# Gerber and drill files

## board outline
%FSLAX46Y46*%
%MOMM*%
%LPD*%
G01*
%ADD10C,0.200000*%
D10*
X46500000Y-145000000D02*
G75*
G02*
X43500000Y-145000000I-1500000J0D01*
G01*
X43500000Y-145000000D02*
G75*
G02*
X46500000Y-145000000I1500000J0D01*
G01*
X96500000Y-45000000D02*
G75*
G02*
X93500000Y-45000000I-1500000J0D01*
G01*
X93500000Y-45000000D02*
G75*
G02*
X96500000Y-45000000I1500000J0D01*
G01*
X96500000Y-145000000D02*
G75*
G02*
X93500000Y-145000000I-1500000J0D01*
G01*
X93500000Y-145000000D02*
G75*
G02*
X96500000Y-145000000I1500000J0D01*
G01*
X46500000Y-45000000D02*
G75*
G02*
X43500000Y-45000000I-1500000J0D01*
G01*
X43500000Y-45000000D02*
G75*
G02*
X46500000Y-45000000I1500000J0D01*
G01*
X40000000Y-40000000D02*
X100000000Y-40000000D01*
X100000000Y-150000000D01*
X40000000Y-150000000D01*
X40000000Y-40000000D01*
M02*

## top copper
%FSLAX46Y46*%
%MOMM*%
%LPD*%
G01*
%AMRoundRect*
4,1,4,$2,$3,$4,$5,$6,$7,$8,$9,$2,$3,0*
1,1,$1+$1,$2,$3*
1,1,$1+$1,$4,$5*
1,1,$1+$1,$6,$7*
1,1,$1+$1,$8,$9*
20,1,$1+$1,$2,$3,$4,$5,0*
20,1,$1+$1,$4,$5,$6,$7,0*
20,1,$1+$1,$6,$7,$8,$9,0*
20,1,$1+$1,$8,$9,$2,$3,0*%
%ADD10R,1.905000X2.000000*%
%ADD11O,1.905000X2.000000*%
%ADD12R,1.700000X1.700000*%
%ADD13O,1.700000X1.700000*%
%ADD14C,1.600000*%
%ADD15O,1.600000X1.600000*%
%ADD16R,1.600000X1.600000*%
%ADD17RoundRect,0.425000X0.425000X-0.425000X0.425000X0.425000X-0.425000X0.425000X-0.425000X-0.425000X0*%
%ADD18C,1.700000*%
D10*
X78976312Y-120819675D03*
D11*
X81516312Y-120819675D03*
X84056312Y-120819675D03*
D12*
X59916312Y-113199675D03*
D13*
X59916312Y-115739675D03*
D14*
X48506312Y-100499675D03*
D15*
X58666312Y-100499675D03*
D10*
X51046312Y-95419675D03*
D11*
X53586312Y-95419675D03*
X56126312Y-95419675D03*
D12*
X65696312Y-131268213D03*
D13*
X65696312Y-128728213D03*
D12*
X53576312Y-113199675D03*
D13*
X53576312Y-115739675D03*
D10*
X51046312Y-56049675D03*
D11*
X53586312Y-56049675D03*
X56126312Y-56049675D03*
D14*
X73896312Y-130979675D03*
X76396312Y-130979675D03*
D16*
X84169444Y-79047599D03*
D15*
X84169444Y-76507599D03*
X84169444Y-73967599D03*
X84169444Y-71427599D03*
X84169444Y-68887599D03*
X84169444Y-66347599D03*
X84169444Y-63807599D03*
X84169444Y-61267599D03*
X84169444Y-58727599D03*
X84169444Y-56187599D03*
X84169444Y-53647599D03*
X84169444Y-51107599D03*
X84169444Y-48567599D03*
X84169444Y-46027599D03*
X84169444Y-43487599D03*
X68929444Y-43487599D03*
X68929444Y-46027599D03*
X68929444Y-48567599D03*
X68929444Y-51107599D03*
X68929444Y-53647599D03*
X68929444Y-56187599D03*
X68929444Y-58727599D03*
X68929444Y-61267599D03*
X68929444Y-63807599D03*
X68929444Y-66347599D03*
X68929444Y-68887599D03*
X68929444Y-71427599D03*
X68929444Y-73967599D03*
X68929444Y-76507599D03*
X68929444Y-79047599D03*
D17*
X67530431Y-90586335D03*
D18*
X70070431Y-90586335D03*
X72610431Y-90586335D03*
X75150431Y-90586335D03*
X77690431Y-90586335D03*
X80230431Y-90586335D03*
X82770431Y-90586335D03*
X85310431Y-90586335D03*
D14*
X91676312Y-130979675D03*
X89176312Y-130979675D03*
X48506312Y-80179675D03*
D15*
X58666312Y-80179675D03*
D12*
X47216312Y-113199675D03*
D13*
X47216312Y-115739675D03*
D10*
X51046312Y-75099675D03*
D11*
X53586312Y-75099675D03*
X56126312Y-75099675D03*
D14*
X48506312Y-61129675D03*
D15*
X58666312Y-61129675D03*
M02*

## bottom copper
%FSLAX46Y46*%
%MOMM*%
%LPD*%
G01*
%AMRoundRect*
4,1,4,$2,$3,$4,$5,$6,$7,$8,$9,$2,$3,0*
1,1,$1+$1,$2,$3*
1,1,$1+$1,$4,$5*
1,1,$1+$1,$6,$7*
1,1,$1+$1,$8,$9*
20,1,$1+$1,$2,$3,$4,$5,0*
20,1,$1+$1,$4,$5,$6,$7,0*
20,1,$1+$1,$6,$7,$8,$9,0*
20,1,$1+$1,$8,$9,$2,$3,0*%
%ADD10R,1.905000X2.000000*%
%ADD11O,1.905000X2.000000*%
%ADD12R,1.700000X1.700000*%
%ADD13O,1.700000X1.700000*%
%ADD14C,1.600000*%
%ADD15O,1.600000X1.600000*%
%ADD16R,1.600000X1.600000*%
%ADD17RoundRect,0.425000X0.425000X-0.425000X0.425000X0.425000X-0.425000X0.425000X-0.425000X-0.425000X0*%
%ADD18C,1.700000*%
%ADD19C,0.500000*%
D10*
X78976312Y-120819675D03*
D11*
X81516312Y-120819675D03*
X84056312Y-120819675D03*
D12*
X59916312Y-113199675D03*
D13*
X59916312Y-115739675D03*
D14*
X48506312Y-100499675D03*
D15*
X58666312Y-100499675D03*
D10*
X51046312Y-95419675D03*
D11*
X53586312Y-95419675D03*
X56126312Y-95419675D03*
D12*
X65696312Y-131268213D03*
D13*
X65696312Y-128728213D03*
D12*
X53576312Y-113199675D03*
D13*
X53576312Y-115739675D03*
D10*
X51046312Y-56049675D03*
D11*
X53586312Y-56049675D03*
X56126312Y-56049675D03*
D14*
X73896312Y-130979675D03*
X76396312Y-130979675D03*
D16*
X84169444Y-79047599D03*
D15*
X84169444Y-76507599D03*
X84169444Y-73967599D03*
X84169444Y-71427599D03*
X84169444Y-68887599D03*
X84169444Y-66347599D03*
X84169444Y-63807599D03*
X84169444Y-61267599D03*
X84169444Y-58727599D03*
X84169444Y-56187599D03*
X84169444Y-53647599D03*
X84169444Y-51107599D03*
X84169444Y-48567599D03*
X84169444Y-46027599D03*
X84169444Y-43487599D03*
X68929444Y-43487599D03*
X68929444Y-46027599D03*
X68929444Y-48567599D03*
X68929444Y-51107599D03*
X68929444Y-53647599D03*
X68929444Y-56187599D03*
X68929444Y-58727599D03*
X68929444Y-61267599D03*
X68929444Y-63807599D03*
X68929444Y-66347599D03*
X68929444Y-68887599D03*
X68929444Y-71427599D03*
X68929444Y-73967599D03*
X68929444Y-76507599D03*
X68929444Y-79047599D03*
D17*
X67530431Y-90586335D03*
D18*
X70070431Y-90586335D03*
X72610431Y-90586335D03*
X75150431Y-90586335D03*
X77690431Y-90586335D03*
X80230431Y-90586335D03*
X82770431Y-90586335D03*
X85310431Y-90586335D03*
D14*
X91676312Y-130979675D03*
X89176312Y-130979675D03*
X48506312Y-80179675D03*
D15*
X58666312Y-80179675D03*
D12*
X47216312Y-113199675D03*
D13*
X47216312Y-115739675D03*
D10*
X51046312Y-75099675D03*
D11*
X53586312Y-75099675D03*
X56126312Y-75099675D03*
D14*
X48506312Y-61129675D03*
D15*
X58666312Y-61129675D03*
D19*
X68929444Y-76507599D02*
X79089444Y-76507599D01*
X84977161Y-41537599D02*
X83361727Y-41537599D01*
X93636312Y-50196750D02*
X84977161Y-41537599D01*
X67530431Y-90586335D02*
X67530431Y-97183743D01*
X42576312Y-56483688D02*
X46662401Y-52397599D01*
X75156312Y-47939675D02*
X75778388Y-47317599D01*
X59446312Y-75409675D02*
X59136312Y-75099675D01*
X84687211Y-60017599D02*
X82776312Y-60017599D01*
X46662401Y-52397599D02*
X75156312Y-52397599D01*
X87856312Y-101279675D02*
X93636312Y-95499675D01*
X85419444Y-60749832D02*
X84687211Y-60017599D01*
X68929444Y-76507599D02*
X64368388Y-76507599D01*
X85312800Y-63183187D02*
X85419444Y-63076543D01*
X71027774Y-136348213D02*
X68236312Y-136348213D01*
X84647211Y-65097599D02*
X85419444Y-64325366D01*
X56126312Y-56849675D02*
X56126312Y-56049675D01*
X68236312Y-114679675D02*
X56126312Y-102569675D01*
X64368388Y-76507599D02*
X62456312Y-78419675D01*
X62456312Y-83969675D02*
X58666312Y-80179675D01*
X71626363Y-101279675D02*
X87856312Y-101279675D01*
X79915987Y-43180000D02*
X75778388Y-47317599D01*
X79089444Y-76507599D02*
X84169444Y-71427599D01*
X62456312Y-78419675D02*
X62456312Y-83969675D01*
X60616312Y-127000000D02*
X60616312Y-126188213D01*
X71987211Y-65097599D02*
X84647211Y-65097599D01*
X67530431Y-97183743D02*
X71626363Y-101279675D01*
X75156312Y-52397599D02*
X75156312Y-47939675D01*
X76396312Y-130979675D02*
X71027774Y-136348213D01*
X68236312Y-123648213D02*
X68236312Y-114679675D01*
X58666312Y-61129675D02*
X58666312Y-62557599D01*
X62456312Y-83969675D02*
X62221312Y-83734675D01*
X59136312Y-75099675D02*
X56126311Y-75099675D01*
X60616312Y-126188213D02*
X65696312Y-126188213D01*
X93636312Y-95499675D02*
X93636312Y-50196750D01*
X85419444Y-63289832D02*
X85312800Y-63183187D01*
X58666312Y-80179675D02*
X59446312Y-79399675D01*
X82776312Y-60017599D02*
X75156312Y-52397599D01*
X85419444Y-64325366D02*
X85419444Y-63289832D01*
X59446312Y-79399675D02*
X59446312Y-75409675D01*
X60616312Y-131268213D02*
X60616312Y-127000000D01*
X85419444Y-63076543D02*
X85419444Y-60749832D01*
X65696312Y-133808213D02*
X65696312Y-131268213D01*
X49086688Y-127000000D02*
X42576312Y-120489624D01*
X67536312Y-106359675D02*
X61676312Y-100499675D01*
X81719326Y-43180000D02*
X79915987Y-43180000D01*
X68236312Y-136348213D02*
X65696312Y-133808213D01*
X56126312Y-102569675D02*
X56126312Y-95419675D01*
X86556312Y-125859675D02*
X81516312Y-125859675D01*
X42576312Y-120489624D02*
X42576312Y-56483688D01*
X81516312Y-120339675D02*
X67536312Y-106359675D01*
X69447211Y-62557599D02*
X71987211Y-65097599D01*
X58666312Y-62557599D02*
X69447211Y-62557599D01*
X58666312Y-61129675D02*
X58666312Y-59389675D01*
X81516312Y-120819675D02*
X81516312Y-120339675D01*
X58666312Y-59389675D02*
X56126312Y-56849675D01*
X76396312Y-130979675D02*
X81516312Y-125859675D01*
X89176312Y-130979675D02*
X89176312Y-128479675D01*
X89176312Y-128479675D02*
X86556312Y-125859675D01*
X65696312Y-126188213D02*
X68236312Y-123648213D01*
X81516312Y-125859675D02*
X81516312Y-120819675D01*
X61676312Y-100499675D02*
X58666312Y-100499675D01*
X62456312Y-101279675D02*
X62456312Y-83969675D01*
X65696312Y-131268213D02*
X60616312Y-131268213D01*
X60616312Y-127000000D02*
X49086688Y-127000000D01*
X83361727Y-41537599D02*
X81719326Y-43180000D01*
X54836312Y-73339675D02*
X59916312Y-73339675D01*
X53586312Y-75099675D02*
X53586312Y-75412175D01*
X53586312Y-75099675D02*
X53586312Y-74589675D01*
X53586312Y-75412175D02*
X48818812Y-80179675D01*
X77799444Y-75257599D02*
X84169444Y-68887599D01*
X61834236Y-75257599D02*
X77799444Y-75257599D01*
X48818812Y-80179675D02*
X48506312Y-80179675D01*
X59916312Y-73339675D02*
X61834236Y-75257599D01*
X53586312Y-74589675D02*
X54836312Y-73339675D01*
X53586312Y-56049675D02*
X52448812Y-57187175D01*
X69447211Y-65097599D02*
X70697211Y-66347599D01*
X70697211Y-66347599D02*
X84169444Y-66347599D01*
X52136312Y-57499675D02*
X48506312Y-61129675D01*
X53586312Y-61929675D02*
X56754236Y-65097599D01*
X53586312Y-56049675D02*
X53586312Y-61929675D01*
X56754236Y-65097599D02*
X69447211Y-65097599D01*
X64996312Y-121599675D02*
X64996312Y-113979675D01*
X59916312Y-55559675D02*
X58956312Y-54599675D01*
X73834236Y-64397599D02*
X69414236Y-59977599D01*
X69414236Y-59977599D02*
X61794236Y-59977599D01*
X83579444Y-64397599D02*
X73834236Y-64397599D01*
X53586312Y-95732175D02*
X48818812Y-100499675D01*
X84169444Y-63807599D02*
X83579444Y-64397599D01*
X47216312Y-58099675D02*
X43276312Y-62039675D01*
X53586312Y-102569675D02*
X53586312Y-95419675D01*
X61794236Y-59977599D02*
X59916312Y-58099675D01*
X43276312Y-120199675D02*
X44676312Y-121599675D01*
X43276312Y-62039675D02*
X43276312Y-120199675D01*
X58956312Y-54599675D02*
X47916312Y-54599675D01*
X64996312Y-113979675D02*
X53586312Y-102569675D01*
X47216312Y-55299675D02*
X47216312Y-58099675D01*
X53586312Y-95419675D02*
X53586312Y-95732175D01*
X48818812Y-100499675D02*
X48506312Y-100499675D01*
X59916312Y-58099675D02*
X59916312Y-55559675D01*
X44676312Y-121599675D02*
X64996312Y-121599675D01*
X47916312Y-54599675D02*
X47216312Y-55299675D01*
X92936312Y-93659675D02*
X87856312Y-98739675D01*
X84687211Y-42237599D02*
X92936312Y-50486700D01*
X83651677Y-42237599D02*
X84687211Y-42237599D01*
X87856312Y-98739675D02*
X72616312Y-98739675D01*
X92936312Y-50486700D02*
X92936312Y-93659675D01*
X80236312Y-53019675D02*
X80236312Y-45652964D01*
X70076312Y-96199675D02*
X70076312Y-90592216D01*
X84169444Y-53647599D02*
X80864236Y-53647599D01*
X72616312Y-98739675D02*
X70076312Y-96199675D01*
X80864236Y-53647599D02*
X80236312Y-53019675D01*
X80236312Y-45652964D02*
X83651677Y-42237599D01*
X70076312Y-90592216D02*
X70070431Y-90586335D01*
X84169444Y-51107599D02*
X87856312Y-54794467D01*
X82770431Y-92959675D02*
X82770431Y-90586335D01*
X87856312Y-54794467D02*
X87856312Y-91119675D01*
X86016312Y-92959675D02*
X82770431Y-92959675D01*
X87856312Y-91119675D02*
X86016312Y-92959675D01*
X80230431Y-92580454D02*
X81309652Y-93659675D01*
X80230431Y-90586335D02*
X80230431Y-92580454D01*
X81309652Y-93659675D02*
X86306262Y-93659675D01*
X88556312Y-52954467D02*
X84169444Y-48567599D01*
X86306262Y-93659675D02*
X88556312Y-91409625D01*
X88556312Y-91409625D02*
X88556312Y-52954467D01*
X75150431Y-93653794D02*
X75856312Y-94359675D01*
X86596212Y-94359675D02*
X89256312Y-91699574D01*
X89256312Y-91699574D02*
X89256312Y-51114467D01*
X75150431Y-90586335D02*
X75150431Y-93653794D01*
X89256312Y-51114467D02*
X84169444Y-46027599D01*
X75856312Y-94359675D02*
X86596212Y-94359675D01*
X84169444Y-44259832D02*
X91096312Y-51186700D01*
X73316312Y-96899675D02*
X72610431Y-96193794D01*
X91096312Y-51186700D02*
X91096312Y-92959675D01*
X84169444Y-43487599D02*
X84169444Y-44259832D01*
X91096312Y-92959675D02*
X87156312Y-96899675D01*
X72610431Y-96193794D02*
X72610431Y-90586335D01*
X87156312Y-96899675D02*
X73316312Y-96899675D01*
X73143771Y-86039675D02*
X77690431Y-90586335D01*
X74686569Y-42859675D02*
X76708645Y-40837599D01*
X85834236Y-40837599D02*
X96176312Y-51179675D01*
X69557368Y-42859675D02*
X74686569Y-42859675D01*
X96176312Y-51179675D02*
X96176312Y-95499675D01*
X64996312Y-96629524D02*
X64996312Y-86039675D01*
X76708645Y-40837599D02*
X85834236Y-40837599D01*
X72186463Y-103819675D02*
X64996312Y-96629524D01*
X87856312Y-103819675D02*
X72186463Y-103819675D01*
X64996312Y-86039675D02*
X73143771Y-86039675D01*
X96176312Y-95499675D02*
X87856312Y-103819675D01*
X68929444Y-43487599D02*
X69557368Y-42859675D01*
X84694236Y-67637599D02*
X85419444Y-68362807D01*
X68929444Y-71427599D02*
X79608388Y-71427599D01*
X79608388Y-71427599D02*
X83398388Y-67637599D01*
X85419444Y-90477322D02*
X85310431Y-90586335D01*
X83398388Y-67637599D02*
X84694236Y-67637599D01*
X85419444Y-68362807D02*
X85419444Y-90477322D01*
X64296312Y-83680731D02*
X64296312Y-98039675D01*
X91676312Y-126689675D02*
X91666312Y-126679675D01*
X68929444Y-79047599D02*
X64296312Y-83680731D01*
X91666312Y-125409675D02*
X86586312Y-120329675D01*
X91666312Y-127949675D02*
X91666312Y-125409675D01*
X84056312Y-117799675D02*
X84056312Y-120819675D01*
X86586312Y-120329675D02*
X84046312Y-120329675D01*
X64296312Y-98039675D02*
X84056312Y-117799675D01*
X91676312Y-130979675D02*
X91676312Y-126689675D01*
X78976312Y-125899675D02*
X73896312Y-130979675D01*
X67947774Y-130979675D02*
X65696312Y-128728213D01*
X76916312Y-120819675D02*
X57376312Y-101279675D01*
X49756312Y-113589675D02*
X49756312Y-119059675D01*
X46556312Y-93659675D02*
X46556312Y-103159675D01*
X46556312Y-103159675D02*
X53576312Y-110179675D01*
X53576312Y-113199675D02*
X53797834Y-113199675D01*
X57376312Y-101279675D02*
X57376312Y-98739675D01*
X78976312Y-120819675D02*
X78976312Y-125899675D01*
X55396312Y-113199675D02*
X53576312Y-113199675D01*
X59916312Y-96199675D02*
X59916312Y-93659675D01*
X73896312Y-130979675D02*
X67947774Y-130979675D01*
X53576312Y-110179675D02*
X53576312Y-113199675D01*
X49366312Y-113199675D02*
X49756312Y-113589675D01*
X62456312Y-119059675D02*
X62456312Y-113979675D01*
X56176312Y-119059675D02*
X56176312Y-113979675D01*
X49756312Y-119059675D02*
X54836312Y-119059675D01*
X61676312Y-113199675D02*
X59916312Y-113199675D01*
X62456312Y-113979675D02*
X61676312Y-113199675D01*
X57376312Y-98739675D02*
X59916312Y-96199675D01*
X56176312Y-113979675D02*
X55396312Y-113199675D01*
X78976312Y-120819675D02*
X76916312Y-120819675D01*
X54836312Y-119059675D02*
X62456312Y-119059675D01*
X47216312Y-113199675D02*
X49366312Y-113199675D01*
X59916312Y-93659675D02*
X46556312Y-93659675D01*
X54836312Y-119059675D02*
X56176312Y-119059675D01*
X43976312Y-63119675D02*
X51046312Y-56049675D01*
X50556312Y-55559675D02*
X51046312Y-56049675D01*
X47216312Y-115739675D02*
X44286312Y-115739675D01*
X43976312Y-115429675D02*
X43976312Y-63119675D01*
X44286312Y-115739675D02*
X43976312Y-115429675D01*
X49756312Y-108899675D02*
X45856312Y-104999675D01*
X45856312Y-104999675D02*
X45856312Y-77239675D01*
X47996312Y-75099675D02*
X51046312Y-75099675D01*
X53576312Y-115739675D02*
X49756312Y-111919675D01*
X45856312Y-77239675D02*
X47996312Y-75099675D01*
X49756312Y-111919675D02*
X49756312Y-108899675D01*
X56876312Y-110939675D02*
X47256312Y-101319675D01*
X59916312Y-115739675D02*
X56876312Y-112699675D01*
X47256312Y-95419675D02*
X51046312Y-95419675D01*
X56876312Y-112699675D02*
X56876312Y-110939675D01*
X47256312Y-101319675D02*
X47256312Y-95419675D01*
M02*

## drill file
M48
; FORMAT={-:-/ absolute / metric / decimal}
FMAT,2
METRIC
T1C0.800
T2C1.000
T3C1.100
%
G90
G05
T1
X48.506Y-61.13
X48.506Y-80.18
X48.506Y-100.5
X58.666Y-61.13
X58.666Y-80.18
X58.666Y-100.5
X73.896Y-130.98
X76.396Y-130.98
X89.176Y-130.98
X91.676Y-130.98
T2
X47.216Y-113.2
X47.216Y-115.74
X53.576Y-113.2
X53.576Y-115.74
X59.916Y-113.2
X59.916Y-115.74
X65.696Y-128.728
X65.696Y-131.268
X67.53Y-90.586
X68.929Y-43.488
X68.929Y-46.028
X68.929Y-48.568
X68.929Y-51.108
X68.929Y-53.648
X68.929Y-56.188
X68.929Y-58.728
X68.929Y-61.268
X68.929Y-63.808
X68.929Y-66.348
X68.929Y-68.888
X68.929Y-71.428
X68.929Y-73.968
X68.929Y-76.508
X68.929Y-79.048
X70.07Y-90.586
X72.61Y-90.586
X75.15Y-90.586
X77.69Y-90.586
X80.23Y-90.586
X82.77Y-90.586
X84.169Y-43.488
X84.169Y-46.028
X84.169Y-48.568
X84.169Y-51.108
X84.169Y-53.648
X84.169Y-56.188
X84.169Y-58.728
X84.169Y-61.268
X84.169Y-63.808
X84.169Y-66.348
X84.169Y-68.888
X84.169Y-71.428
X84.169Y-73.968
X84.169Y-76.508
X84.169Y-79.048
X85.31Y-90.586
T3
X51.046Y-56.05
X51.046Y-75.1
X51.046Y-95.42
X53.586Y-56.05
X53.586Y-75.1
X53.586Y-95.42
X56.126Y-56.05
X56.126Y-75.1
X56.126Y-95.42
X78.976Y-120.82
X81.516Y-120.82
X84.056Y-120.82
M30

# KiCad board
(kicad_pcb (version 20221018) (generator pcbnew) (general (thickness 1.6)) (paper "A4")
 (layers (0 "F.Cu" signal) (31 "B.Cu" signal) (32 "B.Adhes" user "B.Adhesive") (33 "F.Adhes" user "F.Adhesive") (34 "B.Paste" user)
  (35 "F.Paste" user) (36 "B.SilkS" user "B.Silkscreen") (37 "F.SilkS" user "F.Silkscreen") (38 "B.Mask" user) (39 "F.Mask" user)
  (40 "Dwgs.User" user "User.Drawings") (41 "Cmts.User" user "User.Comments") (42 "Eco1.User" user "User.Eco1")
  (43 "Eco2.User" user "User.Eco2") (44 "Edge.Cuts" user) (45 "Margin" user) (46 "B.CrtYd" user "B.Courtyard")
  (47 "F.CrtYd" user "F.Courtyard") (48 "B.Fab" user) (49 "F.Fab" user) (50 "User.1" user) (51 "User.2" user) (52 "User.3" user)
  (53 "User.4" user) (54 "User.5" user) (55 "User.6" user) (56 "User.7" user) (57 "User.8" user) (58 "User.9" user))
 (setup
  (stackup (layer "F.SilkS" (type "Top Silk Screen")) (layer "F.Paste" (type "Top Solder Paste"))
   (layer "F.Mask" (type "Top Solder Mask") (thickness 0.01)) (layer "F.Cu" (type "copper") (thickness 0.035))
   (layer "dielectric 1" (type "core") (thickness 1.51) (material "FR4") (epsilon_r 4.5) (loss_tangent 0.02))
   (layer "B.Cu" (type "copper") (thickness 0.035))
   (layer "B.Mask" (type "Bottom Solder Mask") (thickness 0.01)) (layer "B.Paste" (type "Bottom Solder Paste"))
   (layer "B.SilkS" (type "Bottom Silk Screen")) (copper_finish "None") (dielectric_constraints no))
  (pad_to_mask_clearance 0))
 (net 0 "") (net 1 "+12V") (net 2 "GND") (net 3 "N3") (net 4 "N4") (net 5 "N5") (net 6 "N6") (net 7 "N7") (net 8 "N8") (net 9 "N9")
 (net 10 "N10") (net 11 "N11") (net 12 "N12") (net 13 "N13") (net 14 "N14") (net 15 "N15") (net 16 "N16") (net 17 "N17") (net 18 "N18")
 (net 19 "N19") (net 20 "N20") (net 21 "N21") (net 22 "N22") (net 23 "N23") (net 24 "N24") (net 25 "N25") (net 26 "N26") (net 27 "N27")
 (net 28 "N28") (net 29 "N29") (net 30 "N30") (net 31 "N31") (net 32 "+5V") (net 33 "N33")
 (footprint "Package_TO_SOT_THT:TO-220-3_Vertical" (layer "F.Cu") (at 78.976312 120.819675)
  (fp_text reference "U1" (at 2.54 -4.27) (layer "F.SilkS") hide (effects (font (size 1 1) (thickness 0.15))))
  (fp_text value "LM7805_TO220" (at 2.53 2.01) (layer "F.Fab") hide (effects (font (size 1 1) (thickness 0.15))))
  (pad "1" thru_hole rect (at 0 0) (size 1.905 2) (drill 1.1) (layers "*.Cu" "*.Mask") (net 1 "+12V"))
  (pad "2" thru_hole oval (at 2.54 0) (size 1.905 2) (drill 1.1) (layers "*.Cu" "*.Mask") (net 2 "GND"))
  (pad "3" thru_hole oval (at 5.08 0) (size 1.905 2) (drill 1.1) (layers "*.Cu" "*.Mask") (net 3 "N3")))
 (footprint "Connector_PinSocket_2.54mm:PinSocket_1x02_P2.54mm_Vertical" (layer "F.Cu") (at 59.916312 113.199675)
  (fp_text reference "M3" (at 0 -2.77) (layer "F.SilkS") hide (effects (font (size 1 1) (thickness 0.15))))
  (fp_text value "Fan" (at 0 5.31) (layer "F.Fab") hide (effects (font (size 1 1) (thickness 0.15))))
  (pad "1" thru_hole rect (at 0 0) (size 1.7 1.7) (drill 1) (layers "*.Cu" "*.Mask") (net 1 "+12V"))
  (pad "2" thru_hole oval (at 0 2.54) (size 1.7 1.7) (drill 1) (layers "*.Cu" "*.Mask") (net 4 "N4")))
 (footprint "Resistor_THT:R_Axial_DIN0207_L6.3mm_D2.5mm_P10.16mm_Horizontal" (layer "F.Cu") (at 48.506312 100.499675)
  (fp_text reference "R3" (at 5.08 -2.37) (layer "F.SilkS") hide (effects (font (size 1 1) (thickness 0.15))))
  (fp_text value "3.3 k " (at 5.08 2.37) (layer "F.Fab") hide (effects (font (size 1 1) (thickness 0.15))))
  (pad "1" thru_hole circle (at 0 0) (size 1.6 1.6) (drill 0.8) (layers "*.Cu" "*.Mask") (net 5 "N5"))
  (pad "2" thru_hole oval (at 10.16 0) (size 1.6 1.6) (drill 0.8) (layers "*.Cu" "*.Mask") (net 2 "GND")))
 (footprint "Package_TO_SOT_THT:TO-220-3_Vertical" (layer "F.Cu") (at 51.046312 95.419675)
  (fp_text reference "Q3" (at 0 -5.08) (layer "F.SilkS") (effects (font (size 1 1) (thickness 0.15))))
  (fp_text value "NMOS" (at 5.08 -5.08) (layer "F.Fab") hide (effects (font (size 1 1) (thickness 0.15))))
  (pad "1" thru_hole rect (at 0 0) (size 1.905 2) (drill 1.1) (layers "*.Cu" "*.Mask") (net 4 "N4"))
  (pad "2" thru_hole oval (at 2.54 0) (size 1.905 2) (drill 1.1) (layers "*.Cu" "*.Mask") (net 5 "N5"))
  (pad "3" thru_hole oval (at 5.08 0) (size 1.905 2) (drill 1.1) (layers "*.Cu" "*.Mask") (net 2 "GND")))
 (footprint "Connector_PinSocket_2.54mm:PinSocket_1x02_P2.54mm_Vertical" (layer "F.Cu") (at 65.696312 131.268213 180)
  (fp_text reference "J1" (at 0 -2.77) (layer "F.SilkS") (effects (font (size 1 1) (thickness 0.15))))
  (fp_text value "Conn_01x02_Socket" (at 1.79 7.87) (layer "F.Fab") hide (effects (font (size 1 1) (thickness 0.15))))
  (pad "1" thru_hole rect (at 0 0 180) (size 1.7 1.7) (drill 1) (layers "*.Cu" "*.Mask") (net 2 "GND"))
  (pad "2" thru_hole oval (at 0 2.54 180) (size 1.7 1.7) (drill 1) (layers "*.Cu" "*.Mask") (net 1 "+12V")))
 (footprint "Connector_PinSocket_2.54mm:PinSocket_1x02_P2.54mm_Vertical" (layer "F.Cu") (at 53.576312 113.199675)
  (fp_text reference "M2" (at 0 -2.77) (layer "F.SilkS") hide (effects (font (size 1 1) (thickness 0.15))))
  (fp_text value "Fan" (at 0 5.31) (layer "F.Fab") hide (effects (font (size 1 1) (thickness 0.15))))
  (pad "1" thru_hole rect (at 0 0) (size 1.7 1.7) (drill 1) (layers "*.Cu" "*.Mask") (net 1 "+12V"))
  (pad "2" thru_hole oval (at 0 2.54) (size 1.7 1.7) (drill 1) (layers "*.Cu" "*.Mask") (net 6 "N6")))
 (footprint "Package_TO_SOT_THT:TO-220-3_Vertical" (layer "F.Cu") (at 51.046312 56.049675)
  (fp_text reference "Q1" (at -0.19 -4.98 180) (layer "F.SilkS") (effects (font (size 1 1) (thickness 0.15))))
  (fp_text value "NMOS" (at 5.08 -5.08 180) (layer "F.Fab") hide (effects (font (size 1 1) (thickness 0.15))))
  (pad "1" thru_hole rect (at 0 0) (size 1.905 2) (drill 1.1) (layers "*.Cu" "*.Mask") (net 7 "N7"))
  (pad "2" thru_hole oval (at 2.54 0) (size 1.905 2) (drill 1.1) (layers "*.Cu" "*.Mask") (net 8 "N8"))
  (pad "3" thru_hole oval (at 5.08 0) (size 1.905 2) (drill 1.1) (layers "*.Cu" "*.Mask") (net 2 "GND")))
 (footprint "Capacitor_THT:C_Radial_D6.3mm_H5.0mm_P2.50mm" (layer "F.Cu") (at 73.896312 130.979675)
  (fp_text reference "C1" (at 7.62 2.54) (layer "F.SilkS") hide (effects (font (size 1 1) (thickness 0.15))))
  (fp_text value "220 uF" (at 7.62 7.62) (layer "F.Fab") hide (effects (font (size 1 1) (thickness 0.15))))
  (pad "1" thru_hole circle (at 0 0) (size 1.6 1.6) (drill 0.8) (layers "*.Cu" "*.Mask") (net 1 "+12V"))
  (pad "2" thru_hole circle (at 2.5 0) (size 1.6 1.6) (drill 0.8) (layers "*.Cu" "*.Mask") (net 2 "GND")))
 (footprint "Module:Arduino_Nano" (layer "F.Cu") (at 84.169444 79.047599 180)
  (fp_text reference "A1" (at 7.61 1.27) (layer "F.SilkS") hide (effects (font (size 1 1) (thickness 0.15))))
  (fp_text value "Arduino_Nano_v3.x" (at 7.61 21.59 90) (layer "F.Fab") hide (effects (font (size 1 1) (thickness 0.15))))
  (pad "1" thru_hole rect (at 0 0 180) (size 1.6 1.6) (drill 1) (layers "*.Cu" "*.Mask") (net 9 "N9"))
  (pad "2" thru_hole oval (at 0 2.54 180) (size 1.6 1.6) (drill 1) (layers "*.Cu" "*.Mask") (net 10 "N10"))
  (pad "3" thru_hole oval (at 0 5.08 180) (size 1.6 1.6) (drill 1) (layers "*.Cu" "*.Mask") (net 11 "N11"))
  (pad "4" thru_hole oval (at 0 7.62 180) (size 1.6 1.6) (drill 1) (layers "*.Cu" "*.Mask") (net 2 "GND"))
  (pad "5" thru_hole oval (at 0 10.16 180) (size 1.6 1.6) (drill 1) (layers "*.Cu" "*.Mask") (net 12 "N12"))
  (pad "6" thru_hole oval (at 0 12.7 180) (size 1.6 1.6) (drill 1) (layers "*.Cu" "*.Mask") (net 8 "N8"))
  (pad "7" thru_hole oval (at 0 15.24 180) (size 1.6 1.6) (drill 1) (layers "*.Cu" "*.Mask") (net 5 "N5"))
  (pad "8" thru_hole oval (at 0 17.78 180) (size 1.6 1.6) (drill 1) (layers "*.Cu" "*.Mask") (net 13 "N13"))
  (pad "9" thru_hole oval (at 0 20.32 180) (size 1.6 1.6) (drill 1) (layers "*.Cu" "*.Mask") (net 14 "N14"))
  (pad "10" thru_hole oval (at 0 22.86 180) (size 1.6 1.6) (drill 1) (layers "*.Cu" "*.Mask") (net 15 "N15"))
  (pad "11" thru_hole oval (at 0 25.4 180) (size 1.6 1.6) (drill 1) (layers "*.Cu" "*.Mask") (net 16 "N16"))
  (pad "12" thru_hole oval (at 0 27.94 180) (size 1.6 1.6) (drill 1) (layers "*.Cu" "*.Mask") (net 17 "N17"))
  (pad "13" thru_hole oval (at 0 30.48 180) (size 1.6 1.6) (drill 1) (layers "*.Cu" "*.Mask") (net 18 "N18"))
  (pad "14" thru_hole oval (at 0 33.02 180) (size 1.6 1.6) (drill 1) (layers "*.Cu" "*.Mask") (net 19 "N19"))
  (pad "15" thru_hole oval (at 0 35.56 180) (size 1.6 1.6) (drill 1) (layers "*.Cu" "*.Mask") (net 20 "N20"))
  (pad "16" thru_hole oval (at 15.24 35.56 180) (size 1.6 1.6) (drill 1) (layers "*.Cu" "*.Mask") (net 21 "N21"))
  (pad "17" thru_hole oval (at 15.24 33.02 180) (size 1.6 1.6) (drill 1) (layers "*.Cu" "*.Mask") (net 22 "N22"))
  (pad "18" thru_hole oval (at 15.24 30.48 180) (size 1.6 1.6) (drill 1) (layers "*.Cu" "*.Mask") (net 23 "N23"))
  (pad "19" thru_hole oval (at 15.24 27.94 180) (size 1.6 1.6) (drill 1) (layers "*.Cu" "*.Mask") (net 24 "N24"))
  (pad "20" thru_hole oval (at 15.24 25.4 180) (size 1.6 1.6) (drill 1) (layers "*.Cu" "*.Mask") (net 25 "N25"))
  (pad "21" thru_hole oval (at 15.24 22.86 180) (size 1.6 1.6) (drill 1) (layers "*.Cu" "*.Mask") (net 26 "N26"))
  (pad "22" thru_hole oval (at 15.24 20.32 180) (size 1.6 1.6) (drill 1) (layers "*.Cu" "*.Mask") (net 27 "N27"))
  (pad "23" thru_hole oval (at 15.24 17.78 180) (size 1.6 1.6) (drill 1) (layers "*.Cu" "*.Mask") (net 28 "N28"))
  (pad "24" thru_hole oval (at 15.24 15.24 180) (size 1.6 1.6) (drill 1) (layers "*.Cu" "*.Mask") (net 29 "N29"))
  (pad "25" thru_hole oval (at 15.24 12.7 180) (size 1.6 1.6) (drill 1) (layers "*.Cu" "*.Mask") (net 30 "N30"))
  (pad "26" thru_hole oval (at 15.24 10.16 180) (size 1.6 1.6) (drill 1) (layers "*.Cu" "*.Mask") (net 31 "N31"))
  (pad "27" thru_hole oval (at 15.24 7.62 180) (size 1.6 1.6) (drill 1) (layers "*.Cu" "*.Mask") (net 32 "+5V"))
  (pad "28" thru_hole oval (at 15.24 5.08 180) (size 1.6 1.6) (drill 1) (layers "*.Cu" "*.Mask") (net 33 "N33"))
  (pad "29" thru_hole oval (at 15.24 2.54 180) (size 1.6 1.6) (drill 1) (layers "*.Cu" "*.Mask") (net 2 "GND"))
  (pad "30" thru_hole oval (at 15.24 0 180) (size 1.6 1.6) (drill 1) (layers "*.Cu" "*.Mask") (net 3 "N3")))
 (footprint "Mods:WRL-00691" (layer "F.Cu") (at 67.367186 98.861184 90)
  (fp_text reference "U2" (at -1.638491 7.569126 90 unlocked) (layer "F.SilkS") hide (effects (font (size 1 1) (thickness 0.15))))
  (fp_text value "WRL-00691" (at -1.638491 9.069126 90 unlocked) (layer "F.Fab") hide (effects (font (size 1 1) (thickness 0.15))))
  (pad "1" thru_hole roundrect (at 8.274849 0.163245 90) (size 1.7 1.7) (drill 1) (layers "*.Cu" "*.Mask") (roundrect_rratio 0.25)
   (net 2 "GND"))
  (pad "2" thru_hole circle (at 8.274849 2.703245 90) (size 1.7 1.7) (drill 1) (layers "*.Cu" "*.Mask") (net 16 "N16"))
  (pad "3" thru_hole circle (at 8.274849 5.243245 90) (size 1.7 1.7) (drill 1) (layers "*.Cu" "*.Mask") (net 20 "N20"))
  (pad "4" thru_hole circle (at 8.274849 7.783245 90) (size 1.7 1.7) (drill 1) (layers "*.Cu" "*.Mask") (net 19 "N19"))
  (pad "5" thru_hole circle (at 8.274849 10.323245 90) (size 1.7 1.7) (drill 1) (layers "*.Cu" "*.Mask") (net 21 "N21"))
  (pad "6" thru_hole circle (at 8.274849 12.863245 90) (size 1.7 1.7) (drill 1) (layers "*.Cu" "*.Mask") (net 18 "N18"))
  (pad "7" thru_hole circle (at 8.274849 15.403245 90) (size 1.7 1.7) (drill 1) (layers "*.Cu" "*.Mask") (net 17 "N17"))
  (pad "8" thru_hole circle (at 8.274849 17.943245 90) (size 1.7 1.7) (drill 1) (layers "*.Cu" "*.Mask") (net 32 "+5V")))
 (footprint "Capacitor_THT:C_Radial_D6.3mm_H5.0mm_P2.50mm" (layer "F.Cu") (at 91.676312 130.979675 180)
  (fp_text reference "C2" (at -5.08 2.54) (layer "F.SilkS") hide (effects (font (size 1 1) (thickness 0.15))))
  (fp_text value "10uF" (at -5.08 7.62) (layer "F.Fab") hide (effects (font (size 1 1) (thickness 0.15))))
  (pad "1" thru_hole circle (at 0 0 180) (size 1.6 1.6) (drill 0.8) (layers "*.Cu" "*.Mask") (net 3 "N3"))
  (pad "2" thru_hole circle (at 2.5 0 180) (size 1.6 1.6) (drill 0.8) (layers "*.Cu" "*.Mask") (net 2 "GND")))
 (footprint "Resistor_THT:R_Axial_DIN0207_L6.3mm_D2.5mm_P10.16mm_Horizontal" (layer "F.Cu") (at 48.506312 80.179675)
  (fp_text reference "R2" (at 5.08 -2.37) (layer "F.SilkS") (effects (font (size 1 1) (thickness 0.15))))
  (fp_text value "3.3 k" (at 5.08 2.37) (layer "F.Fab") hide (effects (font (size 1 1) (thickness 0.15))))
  (pad "1" thru_hole circle (at 0 0) (size 1.6 1.6) (drill 0.8) (layers "*.Cu" "*.Mask") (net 12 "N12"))
  (pad "2" thru_hole oval (at 10.16 0) (size 1.6 1.6) (drill 0.8) (layers "*.Cu" "*.Mask") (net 2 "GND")))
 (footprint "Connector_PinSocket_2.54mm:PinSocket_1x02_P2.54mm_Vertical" (layer "F.Cu") (at 47.216312 113.199675)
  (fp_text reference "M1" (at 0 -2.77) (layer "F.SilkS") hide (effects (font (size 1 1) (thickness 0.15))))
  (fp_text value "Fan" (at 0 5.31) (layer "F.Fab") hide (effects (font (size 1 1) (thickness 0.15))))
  (pad "1" thru_hole rect (at 0 0) (size 1.7 1.7) (drill 1) (layers "*.Cu" "*.Mask") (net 1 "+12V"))
  (pad "2" thru_hole oval (at 0 2.54) (size 1.7 1.7) (drill 1) (layers "*.Cu" "*.Mask") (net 7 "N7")))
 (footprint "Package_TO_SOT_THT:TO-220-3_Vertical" (layer "F.Cu") (at 51.046312 75.099675)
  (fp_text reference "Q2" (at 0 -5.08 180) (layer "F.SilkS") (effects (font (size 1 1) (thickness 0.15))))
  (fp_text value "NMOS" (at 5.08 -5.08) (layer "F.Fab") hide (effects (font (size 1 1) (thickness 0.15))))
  (pad "1" thru_hole rect (at 0 0) (size 1.905 2) (drill 1.1) (layers "*.Cu" "*.Mask") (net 6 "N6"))
  (pad "2" thru_hole oval (at 2.54 0) (size 1.905 2) (drill 1.1) (layers "*.Cu" "*.Mask") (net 12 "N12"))
  (pad "3" thru_hole oval (at 5.08 0) (size 1.905 2) (drill 1.1) (layers "*.Cu" "*.Mask") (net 2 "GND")))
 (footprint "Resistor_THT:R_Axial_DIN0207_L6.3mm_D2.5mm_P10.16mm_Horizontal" (layer "F.Cu") (at 48.506312 61.129675)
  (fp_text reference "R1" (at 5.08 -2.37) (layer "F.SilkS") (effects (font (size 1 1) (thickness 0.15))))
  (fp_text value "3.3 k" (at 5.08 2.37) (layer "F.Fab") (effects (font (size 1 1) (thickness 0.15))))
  (pad "1" thru_hole circle (at 0 0) (size 1.6 1.6) (drill 0.8) (layers "*.Cu" "*.Mask") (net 8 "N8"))
  (pad "2" thru_hole oval (at 10.16 0) (size 1.6 1.6) (drill 0.8) (layers "*.Cu" "*.Mask") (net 2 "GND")))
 (gr_circle locked (center 45 145) (end 46.5 145) (stroke (width 0.2) (type solid)) (fill none) (layer "Edge.Cuts"))
 (gr_circle locked (center 95 45) (end 96.5 45) (stroke (width 0.2) (type solid)) (fill none) (layer "Edge.Cuts"))
 (gr_circle locked (center 95 145) (end 96.5 145) (stroke (width 0.2) (type solid)) (fill none) (layer "Edge.Cuts"))
 (gr_circle locked (center 45 45) (end 46.5 45) (stroke (width 0.2) (type solid)) (fill none) (layer "Edge.Cuts"))
 (gr_rect locked (start 40 40) (end 100 150) (stroke (width 0.2) (type default)) (fill none) (layer "Edge.Cuts"))
 (segment (start 68.929444 76.507599) (end 79.089444 76.507599) (width 0.5) (layer "B.Cu") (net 2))
 (segment (start 84.977161 41.537599) (end 83.361727 41.537599) (width 0.5) (layer "B.Cu") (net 2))
 (segment (start 93.636312 50.19675) (end 84.977161 41.537599) (width 0.5) (layer "B.Cu") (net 2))
 (segment (start 67.530431 90.586335) (end 67.530431 97.183743) (width 0.5) (layer "B.Cu") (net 2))
 (segment (start 42.576312 56.483688) (end 46.662401 52.397599) (width 0.5) (layer "B.Cu") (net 2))
 (segment (start 75.156312 47.939675) (end 75.778388 47.317599) (width 0.5) (layer "B.Cu") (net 2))
 (segment (start 59.446312 75.409675) (end 59.136312 75.099675) (width 0.5) (layer "B.Cu") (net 2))
 (segment (start 84.687211 60.017599) (end 82.776312 60.017599) (width 0.5) (layer "B.Cu") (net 2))
 (segment (start 46.662401 52.397599) (end 75.156312 52.397599) (width 0.5) (layer "B.Cu") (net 2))
 (segment (start 87.856312 101.279675) (end 93.636312 95.499675) (width 0.5) (layer "B.Cu") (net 2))
 (segment (start 85.419444 60.749832) (end 84.687211 60.017599) (width 0.5) (layer "B.Cu") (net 2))
 (segment (start 68.929444 76.507599) (end 64.368388 76.507599) (width 0.5) (layer "B.Cu") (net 2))
 (segment (start 85.3128 63.183187) (end 85.419444 63.076543) (width 0.5) (layer "B.Cu") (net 2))
 (segment (start 71.027774 136.348213) (end 68.236312 136.348213) (width 0.5) (layer "B.Cu") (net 2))
 (segment (start 84.647211 65.097599) (end 85.419444 64.325366) (width 0.5) (layer "B.Cu") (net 2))
 (segment (start 56.126312 56.849675) (end 56.126312 56.049675) (width 0.5) (layer "B.Cu") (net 2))
 (segment (start 68.236312 114.679675) (end 56.126312 102.569675) (width 0.5) (layer "B.Cu") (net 2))
 (segment (start 64.368388 76.507599) (end 62.456312 78.419675) (width 0.5) (layer "B.Cu") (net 2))
 (segment (start 62.456312 83.969675) (end 58.666312 80.179675) (width 0.5) (layer "B.Cu") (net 2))
 (segment (start 71.626363 101.279675) (end 87.856312 101.279675) (width 0.5) (layer "B.Cu") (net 2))
 (segment (start 79.915987 43.18) (end 75.778388 47.317599) (width 0.5) (layer "B.Cu") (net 2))
 (segment (start 79.089444 76.507599) (end 84.169444 71.427599) (width 0.5) (layer "B.Cu") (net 2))
 (segment (start 62.456312 78.419675) (end 62.456312 83.969675) (width 0.5) (layer "B.Cu") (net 2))
 (segment (start 60.616312 127) (end 60.616312 126.188213) (width 0.5) (layer "B.Cu") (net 2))
 (segment (start 71.987211 65.097599) (end 84.647211 65.097599) (width 0.5) (layer "B.Cu") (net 2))
 (segment (start 67.530431 97.183743) (end 71.626363 101.279675) (width 0.5) (layer "B.Cu") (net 2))
 (segment (start 75.156312 52.397599) (end 75.156312 47.939675) (width 0.5) (layer "B.Cu") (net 2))
 (segment (start 76.396312 130.979675) (end 71.027774 136.348213) (width 0.5) (layer "B.Cu") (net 2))
 (segment (start 68.236312 123.648213) (end 68.236312 114.679675) (width 0.5) (layer "B.Cu") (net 2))
 (segment (start 58.666312 61.129675) (end 58.666312 62.557599) (width 0.5) (layer "B.Cu") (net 2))
 (segment (start 62.456312 83.969675) (end 62.221312 83.734675) (width 0.5) (layer "B.Cu") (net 2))
 (segment (start 59.136312 75.099675) (end 56.126311 75.099675) (width 0.5) (layer "B.Cu") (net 2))
 (segment (start 60.616312 126.188213) (end 65.696312 126.188213) (width 0.5) (layer "B.Cu") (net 2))
 (segment (start 93.636312 95.499675) (end 93.636312 50.19675) (width 0.5) (layer "B.Cu") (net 2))
 (segment (start 85.419444 63.289832) (end 85.3128 63.183187) (width 0.5) (layer "B.Cu") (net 2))
 (segment (start 58.666312 80.179675) (end 59.446312 79.399675) (width 0.5) (layer "B.Cu") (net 2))
 (segment (start 82.776312 60.017599) (end 75.156312 52.397599) (width 0.5) (layer "B.Cu") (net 2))
 (segment (start 85.419444 64.325366) (end 85.419444 63.289832) (width 0.5) (layer "B.Cu") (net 2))
 (segment (start 59.446312 79.399675) (end 59.446312 75.409675) (width 0.5) (layer "B.Cu") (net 2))
 (segment (start 60.616312 131.268213) (end 60.616312 127) (width 0.5) (layer "B.Cu") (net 2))
 (segment (start 85.419444 63.076543) (end 85.419444 60.749832) (width 0.5) (layer "B.Cu") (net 2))
 (segment (start 65.696312 133.808213) (end 65.696312 131.268213) (width 0.5) (layer "B.Cu") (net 2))
 (segment (start 49.086688 127) (end 42.576312 120.489624) (width 0.5) (layer "B.Cu") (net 2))
 (segment (start 67.536312 106.359675) (end 61.676312 100.499675) (width 0.5) (layer "B.Cu") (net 2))
 (segment (start 81.719326 43.18) (end 79.915987 43.18) (width 0.5) (layer "B.Cu") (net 2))
 (segment (start 68.236312 136.348213) (end 65.696312 133.808213) (width 0.5) (layer "B.Cu") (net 2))
 (segment (start 56.126312 102.569675) (end 56.126312 95.419675) (width 0.5) (layer "B.Cu") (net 2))
 (segment (start 86.556312 125.859675) (end 81.516312 125.859675) (width 0.5) (layer "B.Cu") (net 2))
 (segment (start 42.576312 120.489624) (end 42.576312 56.483688) (width 0.5) (layer "B.Cu") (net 2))
 (segment (start 81.516312 120.339675) (end 67.536312 106.359675) (width 0.5) (layer "B.Cu") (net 2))
 (segment (start 69.447211 62.557599) (end 71.987211 65.097599) (width 0.5) (layer "B.Cu") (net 2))
 (segment (start 58.666312 62.557599) (end 69.447211 62.557599) (width 0.5) (layer "B.Cu") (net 2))
 (segment (start 58.666312 61.129675) (end 58.666312 59.389675) (width 0.5) (layer "B.Cu") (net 2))
 (segment (start 81.516312 120.819675) (end 81.516312 120.339675) (width 0.5) (layer "B.Cu") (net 2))
 (segment (start 58.666312 59.389675) (end 56.126312 56.849675) (width 0.5) (layer "B.Cu") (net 2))
 (segment (start 76.396312 130.979675) (end 81.516312 125.859675) (width 0.5) (layer "B.Cu") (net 2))
 (segment (start 89.176312 130.979675) (end 89.176312 128.479675) (width 0.5) (layer "B.Cu") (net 2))
 (segment (start 89.176312 128.479675) (end 86.556312 125.859675) (width 0.5) (layer "B.Cu") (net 2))
 (segment (start 65.696312 126.188213) (end 68.236312 123.648213) (width 0.5) (layer "B.Cu") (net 2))
 (segment (start 81.516312 125.859675) (end 81.516312 120.819675) (width 0.5) (layer "B.Cu") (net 2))
 (segment (start 61.676312 100.499675) (end 58.666312 100.499675) (width 0.5) (layer "B.Cu") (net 2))
 (segment (start 62.456312 101.279675) (end 62.456312 83.969675) (width 0.5) (layer "B.Cu") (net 2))
 (segment (start 65.696312 131.268213) (end 60.616312 131.268213) (width 0.5) (layer "B.Cu") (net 2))
 (segment (start 60.616312 127) (end 49.086688 127) (width 0.5) (layer "B.Cu") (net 2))
 (segment (start 83.361727 41.537599) (end 81.719326 43.18) (width 0.5) (layer "B.Cu") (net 2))
 (segment (start 54.836312 73.339675) (end 59.916312 73.339675) (width 0.5) (layer "B.Cu") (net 12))
 (segment (start 53.586312 75.099675) (end 53.586312 75.412175) (width 0.5) (layer "B.Cu") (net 12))
 (segment (start 53.586312 75.099675) (end 53.586312 74.589675) (width 0.5) (layer "B.Cu") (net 12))
 (segment (start 53.586312 75.412175) (end 48.818812 80.179675) (width 0.5) (layer "B.Cu") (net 12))
 (segment (start 77.799444 75.257599) (end 84.169444 68.887599) (width 0.5) (layer "B.Cu") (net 12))
 (segment (start 61.834236 75.257599) (end 77.799444 75.257599) (width 0.5) (layer "B.Cu") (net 12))
 (segment (start 48.818812 80.179675) (end 48.506312 80.179675) (width 0.5) (layer "B.Cu") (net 12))
 (segment (start 59.916312 73.339675) (end 61.834236 75.257599) (width 0.5) (layer "B.Cu") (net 12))
 (segment (start 53.586312 74.589675) (end 54.836312 73.339675) (width 0.5) (layer "B.Cu") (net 12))
 (segment (start 53.586312 56.049675) (end 52.448812 57.187175) (width 0.5) (layer "B.Cu") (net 8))
 (segment (start 69.447211 65.097599) (end 70.697211 66.347599) (width 0.5) (layer "B.Cu") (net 8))
 (segment (start 70.697211 66.347599) (end 84.169444 66.347599) (width 0.5) (layer "B.Cu") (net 8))
 (segment (start 52.136312 57.499675) (end 48.506312 61.129675) (width 0.5) (layer "B.Cu") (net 8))
 (segment (start 53.586312 61.929675) (end 56.754236 65.097599) (width 0.5) (layer "B.Cu") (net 8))
 (segment (start 53.586312 56.049675) (end 53.586312 61.929675) (width 0.5) (layer "B.Cu") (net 8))
 (segment (start 56.754236 65.097599) (end 69.447211 65.097599) (width 0.5) (layer "B.Cu") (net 8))
 (segment (start 64.996312 121.599675) (end 64.996312 113.979675) (width 0.5) (layer "B.Cu") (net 5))
 (segment (start 59.916312 55.559675) (end 58.956312 54.599675) (width 0.5) (layer "B.Cu") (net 5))
 (segment (start 73.834236 64.397599) (end 69.414236 59.977599) (width 0.5) (layer "B.Cu") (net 5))
 (segment (start 69.414236 59.977599) (end 61.794236 59.977599) (width 0.5) (layer "B.Cu") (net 5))
 (segment (start 83.579444 64.397599) (end 73.834236 64.397599) (width 0.5) (layer "B.Cu") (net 5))
 (segment (start 53.586312 95.732175) (end 48.818812 100.499675) (width 0.5) (layer "B.Cu") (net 5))
 (segment (start 84.169444 63.807599) (end 83.579444 64.397599) (width 0.5) (layer "B.Cu") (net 5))
 (segment (start 47.216312 58.099675) (end 43.276312 62.039675) (width 0.5) (layer "B.Cu") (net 5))
 (segment (start 53.586312 102.569675) (end 53.586312 95.419675) (width 0.5) (layer "B.Cu") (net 5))
 (segment (start 61.794236 59.977599) (end 59.916312 58.099675) (width 0.5) (layer "B.Cu") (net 5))
 (segment (start 43.276312 120.199675) (end 44.676312 121.599675) (width 0.5) (layer "B.Cu") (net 5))
 (segment (start 43.276312 62.039675) (end 43.276312 120.199675) (width 0.5) (layer "B.Cu") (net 5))
 (segment (start 58.956312 54.599675) (end 47.916312 54.599675) (width 0.5) (layer "B.Cu") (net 5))
 (segment (start 64.996312 113.979675) (end 53.586312 102.569675) (width 0.5) (layer "B.Cu") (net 5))
 (segment (start 47.216312 55.299675) (end 47.216312 58.099675) (width 0.5) (layer "B.Cu") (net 5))
 (segment (start 53.586312 95.419675) (end 53.586312 95.732175) (width 0.5) (layer "B.Cu") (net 5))
 (segment (start 48.818812 100.499675) (end 48.506312 100.499675) (width 0.5) (layer "B.Cu") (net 5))
 (segment (start 59.916312 58.099675) (end 59.916312 55.559675) (width 0.5) (layer "B.Cu") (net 5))
 (segment (start 44.676312 121.599675) (end 64.996312 121.599675) (width 0.5) (layer "B.Cu") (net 5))
 (segment (start 47.916312 54.599675) (end 47.216312 55.299675) (width 0.5) (layer "B.Cu") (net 5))
 (segment (start 92.936312 93.659675) (end 87.856312 98.739675) (width 0.5) (layer "B.Cu") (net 16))
 (segment (start 84.687211 42.237599) (end 92.936312 50.4867) (width 0.5) (layer "B.Cu") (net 16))
 (segment (start 83.651677 42.237599) (end 84.687211 42.237599) (width 0.5) (layer "B.Cu") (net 16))
 (segment (start 87.856312 98.739675) (end 72.616312 98.739675) (width 0.5) (layer "B.Cu") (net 16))
 (segment (start 92.936312 50.4867) (end 92.936312 93.659675) (width 0.5) (layer "B.Cu") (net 16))
 (segment (start 80.236312 53.019675) (end 80.236312 45.652964) (width 0.5) (layer "B.Cu") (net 16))
 (segment (start 70.076312 96.199675) (end 70.076312 90.592216) (width 0.5) (layer "B.Cu") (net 16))
 (segment (start 84.169444 53.647599) (end 80.864236 53.647599) (width 0.5) (layer "B.Cu") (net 16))
 (segment (start 72.616312 98.739675) (end 70.076312 96.199675) (width 0.5) (layer "B.Cu") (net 16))
 (segment (start 80.864236 53.647599) (end 80.236312 53.019675) (width 0.5) (layer "B.Cu") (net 16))
 (segment (start 80.236312 45.652964) (end 83.651677 42.237599) (width 0.5) (layer "B.Cu") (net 16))
 (segment (start 70.076312 90.592216) (end 70.070431 90.586335) (width 0.5) (layer "B.Cu") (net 16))
 (segment (start 84.169444 51.107599) (end 87.856312 54.794467) (width 0.5) (layer "B.Cu") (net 17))
 (segment (start 82.770431 92.959675) (end 82.770431 90.586335) (width 0.5) (layer "B.Cu") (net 17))
 (segment (start 87.856312 54.794467) (end 87.856312 91.119675) (width 0.5) (layer "B.Cu") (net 17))
 (segment (start 86.016312 92.959675) (end 82.770431 92.959675) (width 0.5) (layer "B.Cu") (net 17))
 (segment (start 87.856312 91.119675) (end 86.016312 92.959675) (width 0.5) (layer "B.Cu") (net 17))
 (segment (start 80.230431 92.580454) (end 81.309652 93.659675) (width 0.5) (layer "B.Cu") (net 18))
 (segment (start 80.230431 90.586335) (end 80.230431 92.580454) (width 0.5) (layer "B.Cu") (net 18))
 (segment (start 81.309652 93.659675) (end 86.306262 93.659675) (width 0.5) (layer "B.Cu") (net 18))
 (segment (start 88.556312 52.954467) (end 84.169444 48.567599) (width 0.5) (layer "B.Cu") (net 18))
 (segment (start 86.306262 93.659675) (end 88.556312 91.409625) (width 0.5) (layer "B.Cu") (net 18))
 (segment (start 88.556312 91.409625) (end 88.556312 52.954467) (width 0.5) (layer "B.Cu") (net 18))
 (segment (start 75.150431 93.653794) (end 75.856312 94.359675) (width 0.5) (layer "B.Cu") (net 19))
 (segment (start 86.596212 94.359675) (end 89.256312 91.699574) (width 0.5) (layer "B.Cu") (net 19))
 (segment (start 89.256312 91.699574) (end 89.256312 51.114467) (width 0.5) (layer "B.Cu") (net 19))
 (segment (start 75.150431 90.586335) (end 75.150431 93.653794) (width 0.5) (layer "B.Cu") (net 19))
 (segment (start 89.256312 51.114467) (end 84.169444 46.027599) (width 0.5) (layer "B.Cu") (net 19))
 (segment (start 75.856312 94.359675) (end 86.596212 94.359675) (width 0.5) (layer "B.Cu") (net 19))
 (segment (start 84.169444 44.259832) (end 91.096312 51.1867) (width 0.5) (layer "B.Cu") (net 20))
 (segment (start 73.316312 96.899675) (end 72.610431 96.193794) (width 0.5) (layer "B.Cu") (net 20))
 (segment (start 91.096312 51.1867) (end 91.096312 92.959675) (width 0.5) (layer "B.Cu") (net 20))
 (segment (start 84.169444 43.487599) (end 84.169444 44.259832) (width 0.5) (layer "B.Cu") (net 20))
 (segment (start 91.096312 92.959675) (end 87.156312 96.899675) (width 0.5) (layer "B.Cu") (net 20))
 (segment (start 72.610431 96.193794) (end 72.610431 90.586335) (width 0.5) (layer "B.Cu") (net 20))
 (segment (start 87.156312 96.899675) (end 73.316312 96.899675) (width 0.5) (layer "B.Cu") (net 20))
 (segment (start 73.143771 86.039675) (end 77.690431 90.586335) (width 0.5) (layer "B.Cu") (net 21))
 (segment (start 74.686569 42.859675) (end 76.708645 40.837599) (width 0.5) (layer "B.Cu") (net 21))
 (segment (start 85.834236 40.837599) (end 96.176312 51.179675) (width 0.5) (layer "B.Cu") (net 21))
 (segment (start 69.557368 42.859675) (end 74.686569 42.859675) (width 0.5) (layer "B.Cu") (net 21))
 (segment (start 96.176312 51.179675) (end 96.176312 95.499675) (width 0.5) (layer "B.Cu") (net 21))
 (segment (start 64.996312 96.629524) (end 64.996312 86.039675) (width 0.5) (layer "B.Cu") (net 21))
 (segment (start 76.708645 40.837599) (end 85.834236 40.837599) (width 0.5) (layer "B.Cu") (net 21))
 (segment (start 72.186463 103.819675) (end 64.996312 96.629524) (width 0.5) (layer "B.Cu") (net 21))
 (segment (start 87.856312 103.819675) (end 72.186463 103.819675) (width 0.5) (layer "B.Cu") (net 21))
 (segment (start 64.996312 86.039675) (end 73.143771 86.039675) (width 0.5) (layer "B.Cu") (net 21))
 (segment (start 96.176312 95.499675) (end 87.856312 103.819675) (width 0.5) (layer "B.Cu") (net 21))
 (segment (start 68.929444 43.487599) (end 69.557368 42.859675) (width 0.5) (layer "B.Cu") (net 21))
 (segment (start 84.694236 67.637599) (end 85.419444 68.362807) (width 0.5) (layer "B.Cu") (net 32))
 (segment (start 68.929444 71.427599) (end 79.608388 71.427599) (width 0.5) (layer "B.Cu") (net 32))
 (segment (start 79.608388 71.427599) (end 83.398388 67.637599) (width 0.5) (layer "B.Cu") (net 32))
 (segment (start 85.419444 90.477322) (end 85.310431 90.586335) (width 0.5) (layer "B.Cu") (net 32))
 (segment (start 83.398388 67.637599) (end 84.694236 67.637599) (width 0.5) (layer "B.Cu") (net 32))
 (segment (start 85.419444 68.362807) (end 85.419444 90.477322) (width 0.5) (layer "B.Cu") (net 32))
 (segment (start 64.296312 83.680731) (end 64.296312 98.039675) (width 0.5) (layer "B.Cu") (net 3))
 (segment (start 91.676312 126.689675) (end 91.666312 126.679675) (width 0.5) (layer "B.Cu") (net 3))
 (segment (start 68.929444 79.047599) (end 64.296312 83.680731) (width 0.5) (layer "B.Cu") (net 3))
 (segment (start 91.666312 125.409675) (end 86.586312 120.329675) (width 0.5) (layer "B.Cu") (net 3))
 (segment (start 91.666312 127.949675) (end 91.666312 125.409675) (width 0.5) (layer "B.Cu") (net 3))
 (segment (start 84.056312 117.799675) (end 84.056312 120.819675) (width 0.5) (layer "B.Cu") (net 3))
 (segment (start 86.586312 120.329675) (end 84.046312 120.329675) (width 0.5) (layer "B.Cu") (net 3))
 (segment (start 64.296312 98.039675) (end 84.056312 117.799675) (width 0.5) (layer "B.Cu") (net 3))
 (segment (start 91.676312 130.979675) (end 91.676312 126.689675) (width 0.5) (layer "B.Cu") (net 3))
 (segment (start 78.976312 125.899675) (end 73.896312 130.979675) (width 0.5) (layer "B.Cu") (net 1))
 (segment (start 67.947774 130.979675) (end 65.696312 128.728213) (width 0.5) (layer "B.Cu") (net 1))
 (segment (start 76.916312 120.819675) (end 57.376312 101.279675) (width 0.5) (layer "B.Cu") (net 1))
 (segment (start 49.756312 113.589675) (end 49.756312 119.059675) (width 0.5) (layer "B.Cu") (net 1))
 (segment (start 46.556312 93.659675) (end 46.556312 103.159675) (width 0.5) (layer "B.Cu") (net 1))
 (segment (start 46.556312 103.159675) (end 53.576312 110.179675) (width 0.5) (layer "B.Cu") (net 1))
 (segment (start 53.576312 113.199675) (end 53.797834 113.199675) (width 0.5) (layer "B.Cu") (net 1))
 (segment (start 57.376312 101.279675) (end 57.376312 98.739675) (width 0.5) (layer "B.Cu") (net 1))
 (segment (start 78.976312 120.819675) (end 78.976312 125.899675) (width 0.5) (layer "B.Cu") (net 1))
 (segment (start 55.396312 113.199675) (end 53.576312 113.199675) (width 0.5) (layer "B.Cu") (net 1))
 (segment (start 59.916312 96.199675) (end 59.916312 93.659675) (width 0.5) (layer "B.Cu") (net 1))
 (segment (start 73.896312 130.979675) (end 67.947774 130.979675) (width 0.5) (layer "B.Cu") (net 1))
 (segment (start 53.576312 110.179675) (end 53.576312 113.199675) (width 0.5) (layer "B.Cu") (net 1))
 (segment (start 49.366312 113.199675) (end 49.756312 113.589675) (width 0.5) (layer "B.Cu") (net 1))
 (segment (start 62.456312 119.059675) (end 62.456312 113.979675) (width 0.5) (layer "B.Cu") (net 1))
 (segment (start 56.176312 119.059675) (end 56.176312 113.979675) (width 0.5) (layer "B.Cu") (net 1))
 (segment (start 49.756312 119.059675) (end 54.836312 119.059675) (width 0.5) (layer "B.Cu") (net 1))
 (segment (start 61.676312 113.199675) (end 59.916312 113.199675) (width 0.5) (layer "B.Cu") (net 1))
 (segment (start 62.456312 113.979675) (end 61.676312 113.199675) (width 0.5) (layer "B.Cu") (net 1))
 (segment (start 57.376312 98.739675) (end 59.916312 96.199675) (width 0.5) (layer "B.Cu") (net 1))
 (segment (start 56.176312 113.979675) (end 55.396312 113.199675) (width 0.5) (layer "B.Cu") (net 1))
 (segment (start 78.976312 120.819675) (end 76.916312 120.819675) (width 0.5) (layer "B.Cu") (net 1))
 (segment (start 54.836312 119.059675) (end 62.456312 119.059675) (width 0.5) (layer "B.Cu") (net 1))
 (segment (start 47.216312 113.199675) (end 49.366312 113.199675) (width 0.5) (layer "B.Cu") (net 1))
 (segment (start 59.916312 93.659675) (end 46.556312 93.659675) (width 0.5) (layer "B.Cu") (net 1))
 (segment (start 54.836312 119.059675) (end 56.176312 119.059675) (width 0.5) (layer "B.Cu") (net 1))
 (segment (start 43.976312 63.119675) (end 51.046312 56.049675) (width 0.5) (layer "B.Cu") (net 7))
 (segment (start 50.556312 55.559675) (end 51.046312 56.049675) (width 0.5) (layer "B.Cu") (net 7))
 (segment (start 47.216312 115.739675) (end 44.286312 115.739675) (width 0.5) (layer "B.Cu") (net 7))
 (segment (start 43.976312 115.429675) (end 43.976312 63.119675) (width 0.5) (layer "B.Cu") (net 7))
 (segment (start 44.286312 115.739675) (end 43.976312 115.429675) (width 0.5) (layer "B.Cu") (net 7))
 (segment (start 49.756312 108.899675) (end 45.856312 104.999675) (width 0.5) (layer "B.Cu") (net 6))
 (segment (start 45.856312 104.999675) (end 45.856312 77.239675) (width 0.5) (layer "B.Cu") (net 6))
 (segment (start 47.996312 75.099675) (end 51.046312 75.099675) (width 0.5) (layer "B.Cu") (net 6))
 (segment (start 53.576312 115.739675) (end 49.756312 111.919675) (width 0.5) (layer "B.Cu") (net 6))
 (segment (start 45.856312 77.239675) (end 47.996312 75.099675) (width 0.5) (layer "B.Cu") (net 6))
 (segment (start 49.756312 111.919675) (end 49.756312 108.899675) (width 0.5) (layer "B.Cu") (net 6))
 (segment (start 56.876312 110.939675) (end 47.256312 101.319675) (width 0.5) (layer "B.Cu") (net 4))
 (segment (start 59.916312 115.739675) (end 56.876312 112.699675) (width 0.5) (layer "B.Cu") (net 4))
 (segment (start 47.256312 95.419675) (end 51.046312 95.419675) (width 0.5) (layer "B.Cu") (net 4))
 (segment (start 56.876312 112.699675) (end 56.876312 110.939675) (width 0.5) (layer "B.Cu") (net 4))
 (segment (start 47.256312 101.319675) (end 47.256312 95.419675) (width 0.5) (layer "B.Cu") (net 4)))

